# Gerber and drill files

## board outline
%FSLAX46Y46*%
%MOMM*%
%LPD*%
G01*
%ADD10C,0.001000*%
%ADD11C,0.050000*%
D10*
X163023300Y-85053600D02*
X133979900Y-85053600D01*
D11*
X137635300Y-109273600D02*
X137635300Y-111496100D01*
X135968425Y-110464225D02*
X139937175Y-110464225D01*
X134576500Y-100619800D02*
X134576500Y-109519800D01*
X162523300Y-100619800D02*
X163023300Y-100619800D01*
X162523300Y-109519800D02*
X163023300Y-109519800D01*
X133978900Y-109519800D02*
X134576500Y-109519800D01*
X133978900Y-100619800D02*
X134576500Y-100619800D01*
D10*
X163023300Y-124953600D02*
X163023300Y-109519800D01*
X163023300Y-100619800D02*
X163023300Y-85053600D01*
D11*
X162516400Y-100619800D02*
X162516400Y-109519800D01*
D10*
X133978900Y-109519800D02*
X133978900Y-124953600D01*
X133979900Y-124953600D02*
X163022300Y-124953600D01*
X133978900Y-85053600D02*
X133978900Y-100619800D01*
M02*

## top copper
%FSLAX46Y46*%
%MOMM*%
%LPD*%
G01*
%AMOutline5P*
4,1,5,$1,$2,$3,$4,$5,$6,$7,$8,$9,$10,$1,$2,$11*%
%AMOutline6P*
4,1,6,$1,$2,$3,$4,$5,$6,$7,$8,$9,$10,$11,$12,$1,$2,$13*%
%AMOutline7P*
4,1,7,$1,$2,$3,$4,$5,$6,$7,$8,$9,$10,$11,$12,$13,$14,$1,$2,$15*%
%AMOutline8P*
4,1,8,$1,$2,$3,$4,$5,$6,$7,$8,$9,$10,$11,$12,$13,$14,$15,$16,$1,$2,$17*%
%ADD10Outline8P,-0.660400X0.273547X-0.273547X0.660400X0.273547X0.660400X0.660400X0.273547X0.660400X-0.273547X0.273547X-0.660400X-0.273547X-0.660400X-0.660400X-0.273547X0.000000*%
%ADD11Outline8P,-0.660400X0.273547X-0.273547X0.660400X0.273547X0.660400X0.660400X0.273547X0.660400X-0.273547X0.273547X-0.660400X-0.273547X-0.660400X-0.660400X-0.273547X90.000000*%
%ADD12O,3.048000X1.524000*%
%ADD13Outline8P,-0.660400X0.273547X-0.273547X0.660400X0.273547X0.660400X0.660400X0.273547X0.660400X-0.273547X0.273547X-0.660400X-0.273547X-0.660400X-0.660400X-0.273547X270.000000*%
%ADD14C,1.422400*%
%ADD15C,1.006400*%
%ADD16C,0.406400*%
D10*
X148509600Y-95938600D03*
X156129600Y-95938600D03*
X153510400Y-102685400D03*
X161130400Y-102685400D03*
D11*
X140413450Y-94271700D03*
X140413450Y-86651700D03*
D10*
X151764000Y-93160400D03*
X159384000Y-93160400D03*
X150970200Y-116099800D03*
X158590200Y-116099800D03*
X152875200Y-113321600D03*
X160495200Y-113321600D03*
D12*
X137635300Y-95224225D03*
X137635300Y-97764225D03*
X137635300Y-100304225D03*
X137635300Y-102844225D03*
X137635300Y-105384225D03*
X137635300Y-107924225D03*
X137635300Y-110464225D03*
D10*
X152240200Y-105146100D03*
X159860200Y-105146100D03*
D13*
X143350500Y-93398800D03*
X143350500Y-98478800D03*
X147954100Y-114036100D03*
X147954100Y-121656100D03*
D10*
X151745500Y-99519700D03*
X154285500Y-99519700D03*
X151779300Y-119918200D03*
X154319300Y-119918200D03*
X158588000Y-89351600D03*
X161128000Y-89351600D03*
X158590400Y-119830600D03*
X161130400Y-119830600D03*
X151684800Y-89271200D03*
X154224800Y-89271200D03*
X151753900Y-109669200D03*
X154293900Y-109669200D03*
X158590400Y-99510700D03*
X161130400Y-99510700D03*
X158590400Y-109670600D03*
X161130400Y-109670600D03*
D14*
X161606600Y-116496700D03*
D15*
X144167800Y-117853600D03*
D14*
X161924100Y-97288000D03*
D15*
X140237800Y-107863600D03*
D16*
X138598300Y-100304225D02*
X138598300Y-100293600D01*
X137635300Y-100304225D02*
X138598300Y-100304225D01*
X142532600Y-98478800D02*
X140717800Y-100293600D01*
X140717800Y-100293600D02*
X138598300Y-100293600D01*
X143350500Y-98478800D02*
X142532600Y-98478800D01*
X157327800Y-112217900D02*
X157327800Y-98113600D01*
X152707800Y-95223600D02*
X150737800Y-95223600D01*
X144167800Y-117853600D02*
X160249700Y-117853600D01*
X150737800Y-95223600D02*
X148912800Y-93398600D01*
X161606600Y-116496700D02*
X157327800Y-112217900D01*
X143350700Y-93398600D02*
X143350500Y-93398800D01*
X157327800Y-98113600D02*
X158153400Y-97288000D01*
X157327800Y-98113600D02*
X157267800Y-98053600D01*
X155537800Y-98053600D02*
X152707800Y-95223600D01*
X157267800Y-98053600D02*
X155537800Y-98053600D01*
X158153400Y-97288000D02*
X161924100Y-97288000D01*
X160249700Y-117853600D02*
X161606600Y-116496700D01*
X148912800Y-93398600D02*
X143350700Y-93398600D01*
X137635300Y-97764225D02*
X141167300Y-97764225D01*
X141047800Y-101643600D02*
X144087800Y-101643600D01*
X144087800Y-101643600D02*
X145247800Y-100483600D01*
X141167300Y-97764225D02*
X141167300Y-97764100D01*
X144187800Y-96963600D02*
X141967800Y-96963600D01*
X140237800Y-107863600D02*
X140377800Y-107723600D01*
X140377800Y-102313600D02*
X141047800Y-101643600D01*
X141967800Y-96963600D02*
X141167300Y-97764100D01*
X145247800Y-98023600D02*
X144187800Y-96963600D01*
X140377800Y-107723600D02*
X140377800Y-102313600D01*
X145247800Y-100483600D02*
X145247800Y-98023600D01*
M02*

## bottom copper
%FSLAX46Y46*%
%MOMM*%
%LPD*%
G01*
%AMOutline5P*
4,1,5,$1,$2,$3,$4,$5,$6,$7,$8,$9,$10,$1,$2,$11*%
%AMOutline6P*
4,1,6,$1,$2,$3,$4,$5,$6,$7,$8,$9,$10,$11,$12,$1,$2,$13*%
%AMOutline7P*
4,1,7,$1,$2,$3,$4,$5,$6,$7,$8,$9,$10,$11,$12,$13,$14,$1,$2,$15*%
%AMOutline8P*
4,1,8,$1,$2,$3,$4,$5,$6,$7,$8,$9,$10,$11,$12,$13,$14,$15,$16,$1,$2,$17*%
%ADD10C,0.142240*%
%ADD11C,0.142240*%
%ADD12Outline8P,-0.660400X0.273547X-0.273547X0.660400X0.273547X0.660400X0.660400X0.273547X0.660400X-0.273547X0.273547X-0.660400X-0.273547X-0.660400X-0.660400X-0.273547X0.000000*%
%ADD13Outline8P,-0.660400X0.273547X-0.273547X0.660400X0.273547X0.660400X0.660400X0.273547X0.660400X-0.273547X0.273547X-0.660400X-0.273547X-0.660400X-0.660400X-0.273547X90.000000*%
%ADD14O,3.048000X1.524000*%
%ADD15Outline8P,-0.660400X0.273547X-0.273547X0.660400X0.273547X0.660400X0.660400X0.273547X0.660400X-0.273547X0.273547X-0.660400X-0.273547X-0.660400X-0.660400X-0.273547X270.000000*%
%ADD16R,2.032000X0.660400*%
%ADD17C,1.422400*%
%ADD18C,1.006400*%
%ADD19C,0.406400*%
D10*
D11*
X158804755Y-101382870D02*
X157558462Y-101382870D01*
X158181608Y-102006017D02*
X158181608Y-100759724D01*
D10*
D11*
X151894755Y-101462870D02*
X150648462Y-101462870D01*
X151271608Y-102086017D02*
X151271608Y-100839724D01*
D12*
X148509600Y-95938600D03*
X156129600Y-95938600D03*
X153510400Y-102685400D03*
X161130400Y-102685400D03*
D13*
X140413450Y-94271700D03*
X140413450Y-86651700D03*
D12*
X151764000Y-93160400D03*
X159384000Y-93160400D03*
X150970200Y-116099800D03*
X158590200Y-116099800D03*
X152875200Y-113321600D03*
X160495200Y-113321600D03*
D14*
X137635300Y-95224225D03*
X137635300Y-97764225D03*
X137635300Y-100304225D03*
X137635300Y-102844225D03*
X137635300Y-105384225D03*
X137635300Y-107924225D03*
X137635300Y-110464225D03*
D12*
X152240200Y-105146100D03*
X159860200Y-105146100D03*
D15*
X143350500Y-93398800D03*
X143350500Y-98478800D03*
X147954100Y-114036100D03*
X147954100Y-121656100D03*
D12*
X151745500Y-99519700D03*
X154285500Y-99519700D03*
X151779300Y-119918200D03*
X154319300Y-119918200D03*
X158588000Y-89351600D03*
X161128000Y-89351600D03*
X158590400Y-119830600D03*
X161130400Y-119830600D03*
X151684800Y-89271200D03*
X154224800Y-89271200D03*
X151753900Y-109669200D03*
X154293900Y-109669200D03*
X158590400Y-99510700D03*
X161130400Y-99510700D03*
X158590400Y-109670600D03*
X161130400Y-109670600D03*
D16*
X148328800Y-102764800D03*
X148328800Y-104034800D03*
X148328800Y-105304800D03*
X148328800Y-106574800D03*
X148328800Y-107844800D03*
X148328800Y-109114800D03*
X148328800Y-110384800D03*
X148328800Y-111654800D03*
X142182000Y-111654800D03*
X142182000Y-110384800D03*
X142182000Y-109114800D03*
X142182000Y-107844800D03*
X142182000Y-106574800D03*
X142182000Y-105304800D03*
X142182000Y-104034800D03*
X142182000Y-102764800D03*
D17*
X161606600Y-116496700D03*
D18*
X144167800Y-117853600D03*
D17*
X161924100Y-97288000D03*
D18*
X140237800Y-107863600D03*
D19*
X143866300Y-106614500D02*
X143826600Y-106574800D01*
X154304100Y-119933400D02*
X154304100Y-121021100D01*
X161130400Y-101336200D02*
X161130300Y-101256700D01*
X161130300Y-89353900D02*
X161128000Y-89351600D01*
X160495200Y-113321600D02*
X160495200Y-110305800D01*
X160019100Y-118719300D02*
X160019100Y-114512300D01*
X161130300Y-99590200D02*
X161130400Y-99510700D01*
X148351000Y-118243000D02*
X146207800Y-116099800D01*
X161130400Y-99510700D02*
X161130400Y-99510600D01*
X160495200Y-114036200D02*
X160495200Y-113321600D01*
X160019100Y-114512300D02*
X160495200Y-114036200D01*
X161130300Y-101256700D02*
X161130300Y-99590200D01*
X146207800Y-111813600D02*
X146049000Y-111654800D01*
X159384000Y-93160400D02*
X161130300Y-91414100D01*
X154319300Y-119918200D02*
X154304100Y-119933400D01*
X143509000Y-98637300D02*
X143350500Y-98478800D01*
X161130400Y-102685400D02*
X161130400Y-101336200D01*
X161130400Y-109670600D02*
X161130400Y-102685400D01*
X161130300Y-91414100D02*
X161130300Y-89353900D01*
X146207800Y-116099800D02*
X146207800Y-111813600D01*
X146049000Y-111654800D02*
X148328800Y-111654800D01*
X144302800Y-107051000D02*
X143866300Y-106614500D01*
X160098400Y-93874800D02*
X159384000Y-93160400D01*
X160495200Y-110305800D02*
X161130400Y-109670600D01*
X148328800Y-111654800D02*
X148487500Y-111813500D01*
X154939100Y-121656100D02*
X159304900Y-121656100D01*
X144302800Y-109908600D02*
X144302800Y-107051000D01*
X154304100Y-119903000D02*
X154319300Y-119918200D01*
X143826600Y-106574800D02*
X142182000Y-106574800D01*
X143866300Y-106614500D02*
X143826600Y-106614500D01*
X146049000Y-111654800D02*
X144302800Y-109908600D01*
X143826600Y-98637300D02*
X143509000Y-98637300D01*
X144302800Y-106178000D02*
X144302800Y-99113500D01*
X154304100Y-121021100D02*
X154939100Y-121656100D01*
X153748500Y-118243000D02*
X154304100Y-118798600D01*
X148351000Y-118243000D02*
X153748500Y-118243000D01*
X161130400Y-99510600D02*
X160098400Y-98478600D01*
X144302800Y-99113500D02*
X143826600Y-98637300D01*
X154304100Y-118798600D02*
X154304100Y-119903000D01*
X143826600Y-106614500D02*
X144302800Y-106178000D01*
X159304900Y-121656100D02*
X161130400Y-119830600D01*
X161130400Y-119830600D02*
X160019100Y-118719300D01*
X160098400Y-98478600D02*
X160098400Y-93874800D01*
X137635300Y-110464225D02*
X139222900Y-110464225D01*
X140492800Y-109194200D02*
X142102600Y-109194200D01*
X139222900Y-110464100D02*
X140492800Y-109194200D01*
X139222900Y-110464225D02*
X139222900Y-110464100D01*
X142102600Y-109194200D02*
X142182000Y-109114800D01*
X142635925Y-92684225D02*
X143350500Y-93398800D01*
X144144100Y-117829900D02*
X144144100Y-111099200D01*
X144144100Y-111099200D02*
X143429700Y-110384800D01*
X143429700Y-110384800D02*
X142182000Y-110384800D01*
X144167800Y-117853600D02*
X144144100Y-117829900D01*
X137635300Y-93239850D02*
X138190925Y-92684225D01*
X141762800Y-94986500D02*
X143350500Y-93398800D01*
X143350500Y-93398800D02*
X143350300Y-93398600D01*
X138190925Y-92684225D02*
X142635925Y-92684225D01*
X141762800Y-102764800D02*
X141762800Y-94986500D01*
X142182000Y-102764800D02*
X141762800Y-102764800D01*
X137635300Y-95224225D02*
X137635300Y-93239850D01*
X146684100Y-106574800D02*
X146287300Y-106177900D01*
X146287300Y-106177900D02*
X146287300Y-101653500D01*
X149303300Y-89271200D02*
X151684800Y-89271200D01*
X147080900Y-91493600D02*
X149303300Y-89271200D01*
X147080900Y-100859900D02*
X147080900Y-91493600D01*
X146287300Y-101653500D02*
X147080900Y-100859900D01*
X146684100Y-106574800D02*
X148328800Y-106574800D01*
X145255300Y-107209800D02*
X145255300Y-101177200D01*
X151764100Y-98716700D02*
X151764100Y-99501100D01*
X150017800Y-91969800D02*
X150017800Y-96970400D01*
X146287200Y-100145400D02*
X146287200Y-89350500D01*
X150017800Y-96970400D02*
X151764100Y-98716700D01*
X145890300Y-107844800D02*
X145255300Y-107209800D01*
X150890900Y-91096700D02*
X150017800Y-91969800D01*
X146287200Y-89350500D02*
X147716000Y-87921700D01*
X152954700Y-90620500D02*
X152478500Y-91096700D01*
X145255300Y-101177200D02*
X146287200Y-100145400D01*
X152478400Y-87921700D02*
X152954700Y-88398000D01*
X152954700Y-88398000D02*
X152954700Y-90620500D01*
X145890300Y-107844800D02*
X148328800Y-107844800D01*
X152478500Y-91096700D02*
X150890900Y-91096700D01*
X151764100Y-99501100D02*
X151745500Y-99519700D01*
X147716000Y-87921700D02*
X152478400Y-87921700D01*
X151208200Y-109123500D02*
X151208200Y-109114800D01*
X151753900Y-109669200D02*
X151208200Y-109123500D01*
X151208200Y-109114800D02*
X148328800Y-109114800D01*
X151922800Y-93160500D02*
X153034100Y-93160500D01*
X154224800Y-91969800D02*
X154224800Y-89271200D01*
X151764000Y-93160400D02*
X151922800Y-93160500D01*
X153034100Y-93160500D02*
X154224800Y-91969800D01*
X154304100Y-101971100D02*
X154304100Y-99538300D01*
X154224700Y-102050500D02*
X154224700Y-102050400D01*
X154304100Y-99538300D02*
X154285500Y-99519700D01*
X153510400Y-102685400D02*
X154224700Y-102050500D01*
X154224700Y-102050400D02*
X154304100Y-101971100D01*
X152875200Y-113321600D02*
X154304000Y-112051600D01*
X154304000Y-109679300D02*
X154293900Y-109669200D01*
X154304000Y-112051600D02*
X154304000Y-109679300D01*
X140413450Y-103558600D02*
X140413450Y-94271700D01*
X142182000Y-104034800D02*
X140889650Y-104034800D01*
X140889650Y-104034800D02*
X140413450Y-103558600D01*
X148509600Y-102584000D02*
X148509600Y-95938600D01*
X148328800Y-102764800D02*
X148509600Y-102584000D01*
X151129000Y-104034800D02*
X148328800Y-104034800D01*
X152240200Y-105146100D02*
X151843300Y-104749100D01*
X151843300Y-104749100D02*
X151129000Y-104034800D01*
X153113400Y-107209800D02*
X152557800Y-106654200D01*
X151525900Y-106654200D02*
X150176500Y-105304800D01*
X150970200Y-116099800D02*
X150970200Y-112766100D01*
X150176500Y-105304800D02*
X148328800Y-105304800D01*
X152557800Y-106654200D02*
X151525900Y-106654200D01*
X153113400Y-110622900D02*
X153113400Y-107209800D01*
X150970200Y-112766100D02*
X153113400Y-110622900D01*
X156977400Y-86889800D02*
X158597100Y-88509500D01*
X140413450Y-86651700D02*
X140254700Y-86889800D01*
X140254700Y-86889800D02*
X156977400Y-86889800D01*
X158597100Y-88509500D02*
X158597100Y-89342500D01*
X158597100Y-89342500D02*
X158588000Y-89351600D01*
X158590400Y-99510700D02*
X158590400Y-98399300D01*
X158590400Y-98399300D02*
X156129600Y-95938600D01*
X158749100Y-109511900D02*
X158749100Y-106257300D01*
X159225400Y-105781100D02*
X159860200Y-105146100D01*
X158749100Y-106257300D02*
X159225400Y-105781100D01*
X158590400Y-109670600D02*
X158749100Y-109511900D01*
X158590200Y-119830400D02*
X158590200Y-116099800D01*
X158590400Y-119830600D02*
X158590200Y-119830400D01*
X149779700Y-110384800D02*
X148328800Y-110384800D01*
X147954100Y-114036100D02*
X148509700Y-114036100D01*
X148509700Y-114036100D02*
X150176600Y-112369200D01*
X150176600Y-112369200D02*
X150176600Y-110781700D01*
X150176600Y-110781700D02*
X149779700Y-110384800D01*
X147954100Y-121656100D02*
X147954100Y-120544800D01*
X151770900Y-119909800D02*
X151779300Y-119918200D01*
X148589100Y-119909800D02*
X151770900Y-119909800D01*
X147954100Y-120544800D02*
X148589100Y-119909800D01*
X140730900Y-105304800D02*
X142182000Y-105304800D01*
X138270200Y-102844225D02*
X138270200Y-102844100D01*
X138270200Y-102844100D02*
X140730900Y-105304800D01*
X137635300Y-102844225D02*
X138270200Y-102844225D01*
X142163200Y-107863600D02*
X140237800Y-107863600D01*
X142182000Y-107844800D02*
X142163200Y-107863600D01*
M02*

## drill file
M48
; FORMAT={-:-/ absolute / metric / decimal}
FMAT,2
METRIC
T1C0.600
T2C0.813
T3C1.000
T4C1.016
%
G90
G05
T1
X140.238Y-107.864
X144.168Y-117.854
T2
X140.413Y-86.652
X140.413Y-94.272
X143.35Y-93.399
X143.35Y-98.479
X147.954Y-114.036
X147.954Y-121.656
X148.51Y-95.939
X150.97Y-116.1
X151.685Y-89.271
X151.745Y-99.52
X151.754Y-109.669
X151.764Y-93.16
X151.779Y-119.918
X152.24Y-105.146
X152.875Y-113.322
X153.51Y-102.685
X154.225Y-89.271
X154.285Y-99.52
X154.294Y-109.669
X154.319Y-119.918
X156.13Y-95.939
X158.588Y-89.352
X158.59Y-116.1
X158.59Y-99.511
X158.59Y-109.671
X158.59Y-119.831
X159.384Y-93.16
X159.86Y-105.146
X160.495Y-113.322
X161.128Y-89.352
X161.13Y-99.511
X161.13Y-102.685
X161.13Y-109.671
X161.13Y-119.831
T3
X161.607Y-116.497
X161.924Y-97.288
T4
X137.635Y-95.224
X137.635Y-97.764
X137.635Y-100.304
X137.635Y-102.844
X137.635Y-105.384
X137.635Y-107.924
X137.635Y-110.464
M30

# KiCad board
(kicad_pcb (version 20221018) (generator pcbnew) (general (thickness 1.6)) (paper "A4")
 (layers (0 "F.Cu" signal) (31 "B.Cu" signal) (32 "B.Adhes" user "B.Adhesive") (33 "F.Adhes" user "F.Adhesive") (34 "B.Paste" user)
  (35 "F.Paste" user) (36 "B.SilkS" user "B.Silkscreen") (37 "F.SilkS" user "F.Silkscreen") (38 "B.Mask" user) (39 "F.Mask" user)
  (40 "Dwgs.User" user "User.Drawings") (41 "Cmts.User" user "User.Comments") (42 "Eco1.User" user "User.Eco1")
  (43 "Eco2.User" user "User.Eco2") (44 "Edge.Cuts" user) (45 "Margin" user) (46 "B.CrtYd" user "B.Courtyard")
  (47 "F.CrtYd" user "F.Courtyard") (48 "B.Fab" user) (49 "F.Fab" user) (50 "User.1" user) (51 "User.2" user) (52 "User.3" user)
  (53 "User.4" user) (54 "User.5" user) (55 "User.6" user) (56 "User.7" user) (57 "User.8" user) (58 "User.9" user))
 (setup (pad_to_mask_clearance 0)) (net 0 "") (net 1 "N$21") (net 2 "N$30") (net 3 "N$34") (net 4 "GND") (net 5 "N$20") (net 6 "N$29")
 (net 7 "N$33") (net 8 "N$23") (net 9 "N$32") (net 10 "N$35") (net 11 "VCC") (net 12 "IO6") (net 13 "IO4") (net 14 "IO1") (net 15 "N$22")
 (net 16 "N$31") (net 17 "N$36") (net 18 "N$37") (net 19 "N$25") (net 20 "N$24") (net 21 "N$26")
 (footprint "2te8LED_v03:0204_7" (layer "F.Cu") (at 152.3196 95.9386)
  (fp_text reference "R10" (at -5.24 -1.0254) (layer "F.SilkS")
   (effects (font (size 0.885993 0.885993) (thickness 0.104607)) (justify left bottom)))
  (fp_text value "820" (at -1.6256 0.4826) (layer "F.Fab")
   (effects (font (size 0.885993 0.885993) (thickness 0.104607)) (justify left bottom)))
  (pad "1" thru_hole roundrect (at -3.81 0) (size 1.3208 1.3208) (drill 0.8128) (layers "*.Cu" "*.Mask") (roundrect_rratio 0.25)
   (chamfer_ratio 0.2928932188) (chamfer top_left top_right bottom_left bottom_right) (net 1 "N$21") (solder_mask_margin 0.1016)
   (thermal_bridge_angle 0))
  (pad "2" thru_hole roundrect (at 3.81 0) (size 1.3208 1.3208) (drill 0.8128) (layers "*.Cu" "*.Mask") (roundrect_rratio 0.25)
   (chamfer_ratio 0.2928932188) (chamfer top_left top_right bottom_left bottom_right) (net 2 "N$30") (solder_mask_margin 0.1016)
   (thermal_bridge_angle 0)))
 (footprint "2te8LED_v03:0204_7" (layer "F.Cu") (at 157.3204 102.6854)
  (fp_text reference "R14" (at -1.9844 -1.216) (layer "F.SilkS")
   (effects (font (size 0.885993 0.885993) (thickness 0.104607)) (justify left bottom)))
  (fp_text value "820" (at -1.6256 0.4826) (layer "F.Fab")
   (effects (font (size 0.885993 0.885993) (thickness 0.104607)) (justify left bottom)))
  (pad "1" thru_hole roundrect (at -3.81 0) (size 1.3208 1.3208) (drill 0.8128) (layers "*.Cu" "*.Mask") (roundrect_rratio 0.25)
   (chamfer_ratio 0.2928932188) (chamfer top_left top_right bottom_left bottom_right) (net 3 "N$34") (solder_mask_margin 0.1016)
   (thermal_bridge_angle 0))
  (pad "2" thru_hole roundrect (at 3.81 0) (size 1.3208 1.3208) (drill 0.8128) (layers "*.Cu" "*.Mask") (roundrect_rratio 0.25)
   (chamfer_ratio 0.2928932188) (chamfer top_left top_right bottom_left bottom_right) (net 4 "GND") (solder_mask_margin 0.1016)
   (thermal_bridge_angle 0)))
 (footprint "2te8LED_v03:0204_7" (layer "F.Cu") (at 140.41345 90.4617 90)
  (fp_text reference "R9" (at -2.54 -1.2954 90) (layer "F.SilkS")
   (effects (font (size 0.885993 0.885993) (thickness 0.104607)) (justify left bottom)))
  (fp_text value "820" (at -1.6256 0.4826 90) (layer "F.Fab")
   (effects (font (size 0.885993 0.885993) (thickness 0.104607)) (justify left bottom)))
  (pad "1" thru_hole roundrect (at -3.81 0 90) (size 1.3208 1.3208) (drill 0.8128) (layers "*.Cu" "*.Mask") (roundrect_rratio 0.25)
   (chamfer_ratio 0.2928932188) (chamfer top_left top_right bottom_left bottom_right) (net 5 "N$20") (solder_mask_margin 0.1016)
   (thermal_bridge_angle 0))
  (pad "2" thru_hole roundrect (at 3.81 0 90) (size 1.3208 1.3208) (drill 0.8128) (layers "*.Cu" "*.Mask") (roundrect_rratio 0.25)
   (chamfer_ratio 0.2928932188) (chamfer top_left top_right bottom_left bottom_right) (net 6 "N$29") (solder_mask_margin 0.1016)
   (thermal_bridge_angle 0)))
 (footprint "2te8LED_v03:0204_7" (layer "F.Cu") (at 155.574 93.1604)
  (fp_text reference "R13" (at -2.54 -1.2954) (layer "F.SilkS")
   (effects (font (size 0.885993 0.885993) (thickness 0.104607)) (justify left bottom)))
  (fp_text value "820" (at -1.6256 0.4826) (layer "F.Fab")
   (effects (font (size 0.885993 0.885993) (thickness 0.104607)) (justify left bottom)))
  (pad "1" thru_hole roundrect (at -3.81 0) (size 1.3208 1.3208) (drill 0.8128) (layers "*.Cu" "*.Mask") (roundrect_rratio 0.25)
   (chamfer_ratio 0.2928932188) (chamfer top_left top_right bottom_left bottom_right) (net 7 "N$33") (solder_mask_margin 0.1016)
   (thermal_bridge_angle 0))
  (pad "2" thru_hole roundrect (at 3.81 0) (size 1.3208 1.3208) (drill 0.8128) (layers "*.Cu" "*.Mask") (roundrect_rratio 0.25)
   (chamfer_ratio 0.2928932188) (chamfer top_left top_right bottom_left bottom_right) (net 4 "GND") (solder_mask_margin 0.1016)
   (thermal_bridge_angle 0)))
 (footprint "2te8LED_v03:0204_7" (layer "F.Cu") (at 154.7802 116.0998)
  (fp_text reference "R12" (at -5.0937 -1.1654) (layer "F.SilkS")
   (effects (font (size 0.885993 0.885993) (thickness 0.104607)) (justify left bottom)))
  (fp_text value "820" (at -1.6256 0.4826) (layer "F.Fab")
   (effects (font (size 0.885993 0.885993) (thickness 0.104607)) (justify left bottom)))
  (pad "1" thru_hole roundrect (at -3.81 0) (size 1.3208 1.3208) (drill 0.8128) (layers "*.Cu" "*.Mask") (roundrect_rratio 0.25)
   (chamfer_ratio 0.2928932188) (chamfer top_left top_right bottom_left bottom_right) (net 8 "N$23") (solder_mask_margin 0.1016)
   (thermal_bridge_angle 0))
  (pad "2" thru_hole roundrect (at 3.81 0) (size 1.3208 1.3208) (drill 0.8128) (layers "*.Cu" "*.Mask") (roundrect_rratio 0.25)
   (chamfer_ratio 0.2928932188) (chamfer top_left top_right bottom_left bottom_right) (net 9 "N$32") (solder_mask_margin 0.1016)
   (thermal_bridge_angle 0)))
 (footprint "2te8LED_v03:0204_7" (layer "F.Cu") (at 156.6852 113.3216)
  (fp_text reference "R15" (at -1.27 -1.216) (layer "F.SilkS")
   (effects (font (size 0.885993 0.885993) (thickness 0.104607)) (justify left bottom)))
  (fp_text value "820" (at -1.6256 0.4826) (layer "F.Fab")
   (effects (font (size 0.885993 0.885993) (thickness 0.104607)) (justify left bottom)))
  (pad "1" thru_hole roundrect (at -3.81 0) (size 1.3208 1.3208) (drill 0.8128) (layers "*.Cu" "*.Mask") (roundrect_rratio 0.25)
   (chamfer_ratio 0.2928932188) (chamfer top_left top_right bottom_left bottom_right) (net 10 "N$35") (solder_mask_margin 0.1016)
   (thermal_bridge_angle 0))
  (pad "2" thru_hole roundrect (at 3.81 0) (size 1.3208 1.3208) (drill 0.8128) (layers "*.Cu" "*.Mask") (roundrect_rratio 0.25)
   (chamfer_ratio 0.2928932188) (chamfer top_left top_right bottom_left bottom_right) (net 4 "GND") (solder_mask_margin 0.1016)
   (thermal_bridge_angle 0)))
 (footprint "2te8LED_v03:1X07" (layer "F.Cu") (at 137.6353 102.844225 -90)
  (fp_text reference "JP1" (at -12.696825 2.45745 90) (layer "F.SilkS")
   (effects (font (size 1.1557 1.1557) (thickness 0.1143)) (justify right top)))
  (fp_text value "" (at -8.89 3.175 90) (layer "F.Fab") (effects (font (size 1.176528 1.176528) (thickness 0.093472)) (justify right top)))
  (pad "1" thru_hole oval (at -7.62 0) (size 3.048 1.524) (drill 1.016) (layers "*.Cu" "*.Mask") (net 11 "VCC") (solder_mask_margin 0.1016)
   (thermal_bridge_angle 0))
  (pad "2" thru_hole oval (at -5.08 0) (size 3.048 1.524) (drill 1.016) (layers "*.Cu" "*.Mask") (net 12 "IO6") (solder_mask_margin 0.1016)
   (thermal_bridge_angle 0))
  (pad "3" thru_hole oval (at -2.54 0) (size 3.048 1.524) (drill 1.016) (layers "*.Cu" "*.Mask") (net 4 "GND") (solder_mask_margin 0.1016)
   (thermal_bridge_angle 0))
  (pad "4" thru_hole oval (at 0 0) (size 3.048 1.524) (drill 1.016) (layers "*.Cu" "*.Mask") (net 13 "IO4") (solder_mask_margin 0.1016)
   (thermal_bridge_angle 0))
  (pad "5" thru_hole oval (at 2.54 0) (size 3.048 1.524) (drill 1.016) (layers "*.Cu" "*.Mask") (solder_mask_margin 0.1016)
   (thermal_bridge_angle 0))
  (pad "6" thru_hole oval (at 5.08 0) (size 3.048 1.524) (drill 1.016) (layers "*.Cu" "*.Mask") (solder_mask_margin 0.1016)
   (thermal_bridge_angle 0))
  (pad "7" thru_hole oval (at 7.62 0) (size 3.048 1.524) (drill 1.016) (layers "*.Cu" "*.Mask") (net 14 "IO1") (solder_mask_margin 0.1016)
   (thermal_bridge_angle 0)))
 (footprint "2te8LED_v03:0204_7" (layer "F.Cu") (at 156.0502 105.1461)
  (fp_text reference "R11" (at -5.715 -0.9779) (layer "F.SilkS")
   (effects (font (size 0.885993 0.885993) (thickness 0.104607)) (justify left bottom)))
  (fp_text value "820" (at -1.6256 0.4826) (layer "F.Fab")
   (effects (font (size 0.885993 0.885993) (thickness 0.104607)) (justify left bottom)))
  (pad "1" thru_hole roundrect (at -3.81 0) (size 1.3208 1.3208) (drill 0.8128) (layers "*.Cu" "*.Mask") (roundrect_rratio 0.25)
   (chamfer_ratio 0.2928932188) (chamfer top_left top_right bottom_left bottom_right) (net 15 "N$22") (solder_mask_margin 0.1016)
   (thermal_bridge_angle 0))
  (pad "2" thru_hole roundrect (at 3.81 0) (size 1.3208 1.3208) (drill 0.8128) (layers "*.Cu" "*.Mask") (roundrect_rratio 0.25)
   (chamfer_ratio 0.2928932188) (chamfer top_left top_right bottom_left bottom_right) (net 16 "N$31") (solder_mask_margin 0.1016)
   (thermal_bridge_angle 0)))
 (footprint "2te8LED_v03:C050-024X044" (layer "F.Cu") (at 143.3505 95.9388 -90)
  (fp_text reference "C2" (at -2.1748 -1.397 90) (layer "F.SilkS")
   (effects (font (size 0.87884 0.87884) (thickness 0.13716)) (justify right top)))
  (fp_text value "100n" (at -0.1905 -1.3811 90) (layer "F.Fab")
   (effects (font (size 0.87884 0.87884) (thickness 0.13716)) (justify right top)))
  (pad "1" thru_hole roundrect (at -2.54 0 270) (size 1.3208 1.3208) (drill 0.8128) (layers "*.Cu" "*.Mask") (roundrect_rratio 0.25)
   (chamfer_ratio 0.2928932188) (chamfer top_left top_right bottom_left bottom_right) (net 11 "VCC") (solder_mask_margin 0.1016)
   (thermal_bridge_angle 0))
  (pad "2" thru_hole roundrect (at 2.54 0 270) (size 1.3208 1.3208) (drill 0.8128) (layers "*.Cu" "*.Mask") (roundrect_rratio 0.25)
   (chamfer_ratio 0.2928932188) (chamfer top_left top_right bottom_left bottom_right) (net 4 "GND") (solder_mask_margin 0.1016)
   (thermal_bridge_angle 0)))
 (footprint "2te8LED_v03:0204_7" (layer "F.Cu") (at 147.9541 117.8461 -90)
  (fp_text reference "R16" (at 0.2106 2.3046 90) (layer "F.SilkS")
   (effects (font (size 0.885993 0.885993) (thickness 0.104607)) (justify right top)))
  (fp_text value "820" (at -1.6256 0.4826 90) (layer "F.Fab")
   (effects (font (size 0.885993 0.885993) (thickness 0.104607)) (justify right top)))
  (pad "1" thru_hole roundrect (at -3.81 0 270) (size 1.3208 1.3208) (drill 0.8128) (layers "*.Cu" "*.Mask") (roundrect_rratio 0.25)
   (chamfer_ratio 0.2928932188) (chamfer top_left top_right bottom_left bottom_right) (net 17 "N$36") (solder_mask_margin 0.1016)
   (thermal_bridge_angle 0))
  (pad "2" thru_hole roundrect (at 3.81 0 270) (size 1.3208 1.3208) (drill 0.8128) (layers "*.Cu" "*.Mask") (roundrect_rratio 0.25)
   (chamfer_ratio 0.2928932188) (chamfer top_left top_right bottom_left bottom_right) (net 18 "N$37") (solder_mask_margin 0.1016)
   (thermal_bridge_angle 0)))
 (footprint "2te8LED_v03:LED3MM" (layer "B.Cu") (at 153.0155 99.5197)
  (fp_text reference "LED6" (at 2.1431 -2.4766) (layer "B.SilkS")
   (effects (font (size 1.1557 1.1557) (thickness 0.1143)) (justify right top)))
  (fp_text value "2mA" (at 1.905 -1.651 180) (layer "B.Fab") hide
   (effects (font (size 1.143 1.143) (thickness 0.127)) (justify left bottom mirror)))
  (pad "A" thru_hole roundrect (at -1.27 0) (size 1.3208 1.3208) (drill 0.8128) (layers "*.Cu" "*.Mask") (roundrect_rratio 0.25)
   (chamfer_ratio 0.2928932188) (chamfer top_left top_right bottom_left bottom_right) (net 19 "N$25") (solder_mask_margin 0.1016)
   (thermal_bridge_angle 0))
  (pad "K" thru_hole roundrect (at 1.27 0) (size 1.3208 1.3208) (drill 0.8128) (layers "*.Cu" "*.Mask") (roundrect_rratio 0.25)
   (chamfer_ratio 0.2928932188) (chamfer top_left top_right bottom_left bottom_right) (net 3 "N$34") (solder_mask_margin 0.1016)
   (thermal_bridge_angle 0)))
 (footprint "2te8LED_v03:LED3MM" (layer "B.Cu") (at 153.0493 119.9182)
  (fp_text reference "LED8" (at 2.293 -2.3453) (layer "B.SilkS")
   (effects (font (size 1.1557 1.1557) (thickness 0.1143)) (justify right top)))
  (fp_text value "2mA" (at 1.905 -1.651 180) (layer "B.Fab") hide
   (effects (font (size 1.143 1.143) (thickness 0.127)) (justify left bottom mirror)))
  (pad "A" thru_hole roundrect (at -1.27 0) (size 1.3208 1.3208) (drill 0.8128) (layers "*.Cu" "*.Mask") (roundrect_rratio 0.25)
   (chamfer_ratio 0.2928932188) (chamfer top_left top_right bottom_left bottom_right) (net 18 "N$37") (solder_mask_margin 0.1016)
   (thermal_bridge_angle 0))
  (pad "K" thru_hole roundrect (at 1.27 0) (size 1.3208 1.3208) (drill 0.8128) (layers "*.Cu" "*.Mask") (roundrect_rratio 0.25)
   (chamfer_ratio 0.2928932188) (chamfer top_left top_right bottom_left bottom_right) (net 4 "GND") (solder_mask_margin 0.1016)
   (thermal_bridge_angle 0)))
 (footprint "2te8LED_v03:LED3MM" (layer "B.Cu") (at 159.858 89.3516)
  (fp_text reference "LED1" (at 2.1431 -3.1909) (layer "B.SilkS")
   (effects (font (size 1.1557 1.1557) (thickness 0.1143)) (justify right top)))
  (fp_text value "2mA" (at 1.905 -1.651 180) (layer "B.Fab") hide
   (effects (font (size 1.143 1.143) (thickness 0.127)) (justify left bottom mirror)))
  (pad "A" thru_hole roundrect (at -1.27 0) (size 1.3208 1.3208) (drill 0.8128) (layers "*.Cu" "*.Mask") (roundrect_rratio 0.25)
   (chamfer_ratio 0.2928932188) (chamfer top_left top_right bottom_left bottom_right) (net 6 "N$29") (solder_mask_margin 0.1016)
   (thermal_bridge_angle 0))
  (pad "K" thru_hole roundrect (at 1.27 0) (size 1.3208 1.3208) (drill 0.8128) (layers "*.Cu" "*.Mask") (roundrect_rratio 0.25)
   (chamfer_ratio 0.2928932188) (chamfer top_left top_right bottom_left bottom_right) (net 4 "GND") (solder_mask_margin 0.1016)
   (thermal_bridge_angle 0)))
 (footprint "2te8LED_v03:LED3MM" (layer "B.Cu") (at 159.8604 119.8306)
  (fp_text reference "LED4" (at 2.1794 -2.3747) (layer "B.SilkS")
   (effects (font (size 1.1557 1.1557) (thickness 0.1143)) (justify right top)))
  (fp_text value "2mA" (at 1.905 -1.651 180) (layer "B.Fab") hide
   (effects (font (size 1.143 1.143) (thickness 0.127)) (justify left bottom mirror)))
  (pad "A" thru_hole roundrect (at -1.27 0) (size 1.3208 1.3208) (drill 0.8128) (layers "*.Cu" "*.Mask") (roundrect_rratio 0.25)
   (chamfer_ratio 0.2928932188) (chamfer top_left top_right bottom_left bottom_right) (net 9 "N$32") (solder_mask_margin 0.1016)
   (thermal_bridge_angle 0))
  (pad "K" thru_hole roundrect (at 1.27 0) (size 1.3208 1.3208) (drill 0.8128) (layers "*.Cu" "*.Mask") (roundrect_rratio 0.25)
   (chamfer_ratio 0.2928932188) (chamfer top_left top_right bottom_left bottom_right) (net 4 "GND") (solder_mask_margin 0.1016)
   (thermal_bridge_angle 0)))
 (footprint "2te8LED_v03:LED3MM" (layer "B.Cu") (at 152.9548 89.2712)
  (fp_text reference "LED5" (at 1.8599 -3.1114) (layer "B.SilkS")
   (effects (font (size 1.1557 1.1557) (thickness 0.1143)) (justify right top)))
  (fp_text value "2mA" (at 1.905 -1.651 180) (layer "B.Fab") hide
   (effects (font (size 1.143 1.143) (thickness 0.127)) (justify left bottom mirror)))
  (pad "A" thru_hole roundrect (at -1.27 0) (size 1.3208 1.3208) (drill 0.8128) (layers "*.Cu" "*.Mask") (roundrect_rratio 0.25)
   (chamfer_ratio 0.2928932188) (chamfer top_left top_right bottom_left bottom_right) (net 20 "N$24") (solder_mask_margin 0.1016)
   (thermal_bridge_angle 0))
  (pad "K" thru_hole roundrect (at 1.27 0) (size 1.3208 1.3208) (drill 0.8128) (layers "*.Cu" "*.Mask") (roundrect_rratio 0.25)
   (chamfer_ratio 0.2928932188) (chamfer top_left top_right bottom_left bottom_right) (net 7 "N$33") (solder_mask_margin 0.1016)
   (thermal_bridge_angle 0)))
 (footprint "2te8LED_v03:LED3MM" (layer "B.Cu") (at 153.0239 109.6692)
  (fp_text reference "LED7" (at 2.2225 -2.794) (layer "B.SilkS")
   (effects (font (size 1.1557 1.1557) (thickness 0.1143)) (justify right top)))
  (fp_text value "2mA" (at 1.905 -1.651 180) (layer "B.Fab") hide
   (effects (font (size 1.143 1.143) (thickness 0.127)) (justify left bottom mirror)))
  (pad "A" thru_hole roundrect (at -1.27 0) (size 1.3208 1.3208) (drill 0.8128) (layers "*.Cu" "*.Mask") (roundrect_rratio 0.25)
   (chamfer_ratio 0.2928932188) (chamfer top_left top_right bottom_left bottom_right) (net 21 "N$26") (solder_mask_margin 0.1016)
   (thermal_bridge_angle 0))
  (pad "K" thru_hole roundrect (at 1.27 0) (size 1.3208 1.3208) (drill 0.8128) (layers "*.Cu" "*.Mask") (roundrect_rratio 0.25)
   (chamfer_ratio 0.2928932188) (chamfer top_left top_right bottom_left bottom_right) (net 10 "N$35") (solder_mask_margin 0.1016)
   (thermal_bridge_angle 0)))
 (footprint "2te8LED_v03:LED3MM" (layer "B.Cu") (at 159.8604 99.5107)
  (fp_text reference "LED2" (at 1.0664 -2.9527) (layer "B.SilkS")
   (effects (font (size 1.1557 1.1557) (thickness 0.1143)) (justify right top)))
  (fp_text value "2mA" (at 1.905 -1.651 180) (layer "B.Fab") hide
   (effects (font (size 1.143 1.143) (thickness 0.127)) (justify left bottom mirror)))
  (pad "A" thru_hole roundrect (at -1.27 0) (size 1.3208 1.3208) (drill 0.8128) (layers "*.Cu" "*.Mask") (roundrect_rratio 0.25)
   (chamfer_ratio 0.2928932188) (chamfer top_left top_right bottom_left bottom_right) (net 2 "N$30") (solder_mask_margin 0.1016)
   (thermal_bridge_angle 0))
  (pad "K" thru_hole roundrect (at 1.27 0) (size 1.3208 1.3208) (drill 0.8128) (layers "*.Cu" "*.Mask") (roundrect_rratio 0.25)
   (chamfer_ratio 0.2928932188) (chamfer top_left top_right bottom_left bottom_right) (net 4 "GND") (solder_mask_margin 0.1016)
   (thermal_bridge_angle 0)))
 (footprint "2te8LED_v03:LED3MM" (layer "B.Cu") (at 159.8604 109.6706)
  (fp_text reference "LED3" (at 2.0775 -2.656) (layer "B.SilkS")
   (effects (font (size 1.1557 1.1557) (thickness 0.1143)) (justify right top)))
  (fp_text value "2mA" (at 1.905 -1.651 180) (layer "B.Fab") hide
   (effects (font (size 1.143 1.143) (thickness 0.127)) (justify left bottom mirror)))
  (pad "A" thru_hole roundrect (at -1.27 0) (size 1.3208 1.3208) (drill 0.8128) (layers "*.Cu" "*.Mask") (roundrect_rratio 0.25)
   (chamfer_ratio 0.2928932188) (chamfer top_left top_right bottom_left bottom_right) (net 16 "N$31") (solder_mask_margin 0.1016)
   (thermal_bridge_angle 0))
  (pad "K" thru_hole roundrect (at 1.27 0) (size 1.3208 1.3208) (drill 0.8128) (layers "*.Cu" "*.Mask") (roundrect_rratio 0.25)
   (chamfer_ratio 0.2928932188) (chamfer top_left top_right bottom_left bottom_right) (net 4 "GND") (solder_mask_margin 0.1016)
   (thermal_bridge_angle 0)))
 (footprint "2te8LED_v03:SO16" (layer "B.Cu") (at 145.2554 107.2098 -90)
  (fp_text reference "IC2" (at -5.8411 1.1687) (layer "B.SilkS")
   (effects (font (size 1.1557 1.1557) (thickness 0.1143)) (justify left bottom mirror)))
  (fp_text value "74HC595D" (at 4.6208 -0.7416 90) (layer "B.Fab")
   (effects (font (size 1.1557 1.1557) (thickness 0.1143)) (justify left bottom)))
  (pad "1" smd rect (at -4.445 -3.0734 270) (size 0.6604 2.032) (layers "B.Cu" "B.Paste" "B.Mask") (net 1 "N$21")
   (solder_mask_margin 0.1016) (thermal_bridge_angle 0))
  (pad "2" smd rect (at -3.175 -3.0734 270) (size 0.6604 2.032) (layers "B.Cu" "B.Paste" "B.Mask") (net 15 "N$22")
   (solder_mask_margin 0.1016) (thermal_bridge_angle 0))
  (pad "3" smd rect (at -1.905 -3.0734 270) (size 0.6604 2.032) (layers "B.Cu" "B.Paste" "B.Mask") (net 8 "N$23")
   (solder_mask_margin 0.1016) (thermal_bridge_angle 0))
  (pad "4" smd rect (at -0.635 -3.0734 270) (size 0.6604 2.032) (layers "B.Cu" "B.Paste" "B.Mask") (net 20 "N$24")
   (solder_mask_margin 0.1016) (thermal_bridge_angle 0))
  (pad "5" smd rect (at 0.635 -3.0734 270) (size 0.6604 2.032) (layers "B.Cu" "B.Paste" "B.Mask") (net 19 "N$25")
   (solder_mask_margin 0.1016) (thermal_bridge_angle 0))
  (pad "6" smd rect (at 1.905 -3.0734 270) (size 0.6604 2.032) (layers "B.Cu" "B.Paste" "B.Mask") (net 21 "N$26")
   (solder_mask_margin 0.1016) (thermal_bridge_angle 0))
  (pad "7" smd rect (at 3.175 -3.0734 270) (size 0.6604 2.032) (layers "B.Cu" "B.Paste" "B.Mask") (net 17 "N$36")
   (solder_mask_margin 0.1016) (thermal_bridge_angle 0))
  (pad "8" smd rect (at 4.445 -3.0734 270) (size 0.6604 2.032) (layers "B.Cu" "B.Paste" "B.Mask") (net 4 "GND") (solder_mask_margin 0.1016)
   (thermal_bridge_angle 0))
  (pad "9" smd rect (at 4.445 3.0734 270) (size 0.6604 2.032) (layers "B.Cu" "B.Paste" "B.Mask") (solder_mask_margin 0.1016)
   (thermal_bridge_angle 0))
  (pad "10" smd rect (at 3.175 3.0734 270) (size 0.6604 2.032) (layers "B.Cu" "B.Paste" "B.Mask") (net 11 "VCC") (solder_mask_margin 0.1016)
   (thermal_bridge_angle 0))
  (pad "11" smd rect (at 1.905 3.0734 270) (size 0.6604 2.032) (layers "B.Cu" "B.Paste" "B.Mask") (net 14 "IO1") (solder_mask_margin 0.1016)
   (thermal_bridge_angle 0))
  (pad "12" smd rect (at 0.635 3.0734 270) (size 0.6604 2.032) (layers "B.Cu" "B.Paste" "B.Mask") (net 12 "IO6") (solder_mask_margin 0.1016)
   (thermal_bridge_angle 0))
  (pad "13" smd rect (at -0.635 3.0734 270) (size 0.6604 2.032) (layers "B.Cu" "B.Paste" "B.Mask") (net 4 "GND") (solder_mask_margin 0.1016)
   (thermal_bridge_angle 0))
  (pad "14" smd rect (at -1.905 3.0734 270) (size 0.6604 2.032) (layers "B.Cu" "B.Paste" "B.Mask") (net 13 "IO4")
   (solder_mask_margin 0.1016) (thermal_bridge_angle 0))
  (pad "15" smd rect (at -3.175 3.0734 270) (size 0.6604 2.032) (layers "B.Cu" "B.Paste" "B.Mask") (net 5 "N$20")
   (solder_mask_margin 0.1016) (thermal_bridge_angle 0))
  (pad "16" smd rect (at -4.445 3.0734 270) (size 0.6604 2.032) (layers "B.Cu" "B.Paste" "B.Mask") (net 11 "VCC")
   (solder_mask_margin 0.1016) (thermal_bridge_angle 0)))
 (gr_line (start 163.0233 85.0536) (end 133.9799 85.0536) (stroke (width 0.001) (type solid)) (layer "Edge.Cuts"))
 (gr_line (start 137.6353 109.2736) (end 137.6353 111.4961) (stroke (width 0.05) (type solid)) (layer "Edge.Cuts"))
 (gr_line (start 135.968425 110.464225) (end 139.937175 110.464225) (stroke (width 0.05) (type solid)) (layer "Edge.Cuts"))
 (gr_line (start 134.5765 100.6198) (end 134.5765 109.5198) (stroke (width 0.05) (type solid)) (layer "Edge.Cuts"))
 (gr_line (start 162.5233 100.6198) (end 163.0233 100.6198) (stroke (width 0.05) (type solid)) (layer "Edge.Cuts"))
 (gr_line (start 162.5233 109.5198) (end 163.0233 109.5198) (stroke (width 0.05) (type solid)) (layer "Edge.Cuts"))
 (gr_line (start 133.9789 109.5198) (end 134.5765 109.5198) (stroke (width 0.05) (type solid)) (layer "Edge.Cuts"))
 (gr_line (start 133.9789 100.6198) (end 134.5765 100.6198) (stroke (width 0.05) (type solid)) (layer "Edge.Cuts"))
 (gr_line (start 163.0233 124.9536) (end 163.0233 109.5198) (stroke (width 0.001) (type solid)) (layer "Edge.Cuts"))
 (gr_line (start 163.0233 100.6198) (end 163.0233 85.0536) (stroke (width 0.001) (type solid)) (layer "Edge.Cuts"))
 (gr_line (start 162.5164 100.6198) (end 162.5164 109.5198) (stroke (width 0.05) (type solid)) (layer "Edge.Cuts"))
 (gr_line (start 133.9789 109.5198) (end 133.9789 124.9536) (stroke (width 0.001) (type solid)) (layer "Edge.Cuts"))
 (gr_line (start 133.9799 124.9536) (end 163.0223 124.9536) (stroke (width 0.001) (type solid)) (layer "Edge.Cuts"))
 (gr_line (start 133.9789 85.0536) (end 133.9789 100.6198) (stroke (width 0.001) (type solid)) (layer "Edge.Cuts"))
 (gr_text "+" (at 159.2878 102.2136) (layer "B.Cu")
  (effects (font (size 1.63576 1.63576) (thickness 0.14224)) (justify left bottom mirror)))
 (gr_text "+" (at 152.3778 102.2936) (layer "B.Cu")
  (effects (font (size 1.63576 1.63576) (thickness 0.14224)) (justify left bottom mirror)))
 (segment (start 138.5983 100.304225) (end 138.5983 100.2936) (width 0.4064) (layer "F.Cu") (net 4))
 (segment (start 137.6353 100.304225) (end 138.5983 100.304225) (width 0.4064) (layer "F.Cu") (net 4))
 (segment (start 142.5326 98.4788) (end 140.7178 100.2936) (width 0.4064) (layer "F.Cu") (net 4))
 (segment (start 140.7178 100.2936) (end 138.5983 100.2936) (width 0.4064) (layer "F.Cu") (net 4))
 (segment (start 143.3505 98.4788) (end 142.5326 98.4788) (width 0.4064) (layer "F.Cu") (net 4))
 (segment (start 143.8663 106.6145) (end 143.8266 106.5748) (width 0.4064) (layer "B.Cu") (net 4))
 (segment (start 154.3041 119.9334) (end 154.3041 121.0211) (width 0.4064) (layer "B.Cu") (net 4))
 (segment (start 161.1304 101.3362) (end 161.1303 101.2567) (width 0.4064) (layer "B.Cu") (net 4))
 (segment (start 161.1303 89.3539) (end 161.128 89.3516) (width 0.4064) (layer "B.Cu") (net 4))
 (segment (start 160.4952 113.3216) (end 160.4952 110.3058) (width 0.4064) (layer "B.Cu") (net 4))
 (segment (start 160.0191 118.7193) (end 160.0191 114.5123) (width 0.4064) (layer "B.Cu") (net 4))
 (segment (start 161.1303 99.5902) (end 161.1304 99.5107) (width 0.4064) (layer "B.Cu") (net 4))
 (segment (start 148.351 118.243) (end 146.2078 116.0998) (width 0.4064) (layer "B.Cu") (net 4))
 (segment (start 161.1304 99.5107) (end 161.1304 99.5106) (width 0.4064) (layer "B.Cu") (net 4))
 (segment (start 160.4952 114.0362) (end 160.4952 113.3216) (width 0.4064) (layer "B.Cu") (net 4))
 (segment (start 160.0191 114.5123) (end 160.4952 114.0362) (width 0.4064) (layer "B.Cu") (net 4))
 (segment (start 161.1303 101.2567) (end 161.1303 99.5902) (width 0.4064) (layer "B.Cu") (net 4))
 (segment (start 146.2078 111.8136) (end 146.049 111.6548) (width 0.4064) (layer "B.Cu") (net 4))
 (segment (start 159.384 93.1604) (end 161.1303 91.4141) (width 0.4064) (layer "B.Cu") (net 4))
 (segment (start 154.3193 119.9182) (end 154.3041 119.9334) (width 0.4064) (layer "B.Cu") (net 4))
 (segment (start 143.509 98.6373) (end 143.3505 98.4788) (width 0.4064) (layer "B.Cu") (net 4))
 (segment (start 161.1304 102.6854) (end 161.1304 101.3362) (width 0.4064) (layer "B.Cu") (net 4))
 (segment (start 161.1304 109.6706) (end 161.1304 102.6854) (width 0.4064) (layer "B.Cu") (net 4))
 (segment (start 161.1303 91.4141) (end 161.1303 89.3539) (width 0.4064) (layer "B.Cu") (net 4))
 (segment (start 146.2078 116.0998) (end 146.2078 111.8136) (width 0.4064) (layer "B.Cu") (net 4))
 (segment (start 146.049 111.6548) (end 148.3288 111.6548) (width 0.4064) (layer "B.Cu") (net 4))
 (segment (start 144.3028 107.051) (end 143.8663 106.6145) (width 0.4064) (layer "B.Cu") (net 4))
 (segment (start 160.0984 93.8748) (end 159.384 93.1604) (width 0.4064) (layer "B.Cu") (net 4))
 (segment (start 160.4952 110.3058) (end 161.1304 109.6706) (width 0.4064) (layer "B.Cu") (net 4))
 (segment (start 148.3288 111.6548) (end 148.4875 111.8135) (width 0.4064) (layer "B.Cu") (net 4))
 (segment (start 154.9391 121.6561) (end 159.3049 121.6561) (width 0.4064) (layer "B.Cu") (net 4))
 (segment (start 144.3028 109.9086) (end 144.3028 107.051) (width 0.4064) (layer "B.Cu") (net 4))
 (segment (start 154.3041 119.903) (end 154.3193 119.9182) (width 0.4064) (layer "B.Cu") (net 4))
 (segment (start 143.8266 106.5748) (end 142.182 106.5748) (width 0.4064) (layer "B.Cu") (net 4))
 (segment (start 143.8663 106.6145) (end 143.8266 106.6145) (width 0.4064) (layer "B.Cu") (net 4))
 (segment (start 146.049 111.6548) (end 144.3028 109.9086) (width 0.4064) (layer "B.Cu") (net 4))
 (segment (start 143.8266 98.6373) (end 143.509 98.6373) (width 0.4064) (layer "B.Cu") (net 4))
 (segment (start 144.3028 106.178) (end 144.3028 99.1135) (width 0.4064) (layer "B.Cu") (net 4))
 (segment (start 154.3041 121.0211) (end 154.9391 121.6561) (width 0.4064) (layer "B.Cu") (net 4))
 (segment (start 153.7485 118.243) (end 154.3041 118.7986) (width 0.4064) (layer "B.Cu") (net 4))
 (segment (start 148.351 118.243) (end 153.7485 118.243) (width 0.4064) (layer "B.Cu") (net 4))
 (segment (start 161.1304 99.5106) (end 160.0984 98.4786) (width 0.4064) (layer "B.Cu") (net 4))
 (segment (start 144.3028 99.1135) (end 143.8266 98.6373) (width 0.4064) (layer "B.Cu") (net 4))
 (segment (start 154.3041 118.7986) (end 154.3041 119.903) (width 0.4064) (layer "B.Cu") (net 4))
 (segment (start 143.8266 106.6145) (end 144.3028 106.178) (width 0.4064) (layer "B.Cu") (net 4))
 (segment (start 159.3049 121.6561) (end 161.1304 119.8306) (width 0.4064) (layer "B.Cu") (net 4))
 (segment (start 161.1304 119.8306) (end 160.0191 118.7193) (width 0.4064) (layer "B.Cu") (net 4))
 (segment (start 160.0984 98.4786) (end 160.0984 93.8748) (width 0.4064) (layer "B.Cu") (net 4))
 (segment (start 137.6353 110.464225) (end 139.2229 110.464225) (width 0.4064) (layer "B.Cu") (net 14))
 (segment (start 140.4928 109.1942) (end 142.1026 109.1942) (width 0.4064) (layer "B.Cu") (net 14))
 (segment (start 139.2229 110.4641) (end 140.4928 109.1942) (width 0.4064) (layer "B.Cu") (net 14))
 (segment (start 139.2229 110.464225) (end 139.2229 110.4641) (width 0.4064) (layer "B.Cu") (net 14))
 (segment (start 142.1026 109.1942) (end 142.182 109.1148) (width 0.4064) (layer "B.Cu") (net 14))
 (segment (start 157.3278 112.2179) (end 157.3278 98.1136) (width 0.4064) (layer "F.Cu") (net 11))
 (segment (start 152.7078 95.2236) (end 150.7378 95.2236) (width 0.4064) (layer "F.Cu") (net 11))
 (segment (start 144.1678 117.8536) (end 160.2497 117.8536) (width 0.4064) (layer "F.Cu") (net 11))
 (segment (start 150.7378 95.2236) (end 148.9128 93.3986) (width 0.4064) (layer "F.Cu") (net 11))
 (segment (start 161.6066 116.4967) (end 157.3278 112.2179) (width 0.4064) (layer "F.Cu") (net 11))
 (segment (start 143.3507 93.3986) (end 143.3505 93.3988) (width 0.4064) (layer "F.Cu") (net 11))
 (segment (start 157.3278 98.1136) (end 158.1534 97.288) (width 0.4064) (layer "F.Cu") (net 11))
 (segment (start 157.3278 98.1136) (end 157.2678 98.0536) (width 0.4064) (layer "F.Cu") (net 11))
 (segment (start 155.5378 98.0536) (end 152.7078 95.2236) (width 0.4064) (layer "F.Cu") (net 11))
 (segment (start 157.2678 98.0536) (end 155.5378 98.0536) (width 0.4064) (layer "F.Cu") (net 11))
 (segment (start 158.1534 97.288) (end 161.9241 97.288) (width 0.4064) (layer "F.Cu") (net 11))
 (segment (start 160.2497 117.8536) (end 161.6066 116.4967) (width 0.4064) (layer "F.Cu") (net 11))
 (segment (start 148.9128 93.3986) (end 143.3507 93.3986) (width 0.4064) (layer "F.Cu") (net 11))
 (via (at 161.6066 116.4967) (size 1.4224) (drill 1) (layers "F.Cu" "B.Cu") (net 11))
 (via (at 144.1678 117.8536) (size 1.0064) (drill 0.6) (layers "F.Cu" "B.Cu") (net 11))
 (via (at 161.9241 97.288) (size 1.4224) (drill 1) (layers "F.Cu" "B.Cu") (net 11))
 (segment (start 142.635925 92.684225) (end 143.3505 93.3988) (width 0.4064) (layer "B.Cu") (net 11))
 (segment (start 144.1441 117.8299) (end 144.1441 111.0992) (width 0.4064) (layer "B.Cu") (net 11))
 (segment (start 144.1441 111.0992) (end 143.4297 110.3848) (width 0.4064) (layer "B.Cu") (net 11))
 (segment (start 143.4297 110.3848) (end 142.182 110.3848) (width 0.4064) (layer "B.Cu") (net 11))
 (segment (start 144.1678 117.8536) (end 144.1441 117.8299) (width 0.4064) (layer "B.Cu") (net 11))
 (segment (start 137.6353 93.23985) (end 138.190925 92.684225) (width 0.4064) (layer "B.Cu") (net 11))
 (segment (start 141.7628 94.9865) (end 143.3505 93.3988) (width 0.4064) (layer "B.Cu") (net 11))
 (segment (start 143.3505 93.3988) (end 143.3503 93.3986) (width 0.4064) (layer "B.Cu") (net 11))
 (segment (start 138.190925 92.684225) (end 142.635925 92.684225) (width 0.4064) (layer "B.Cu") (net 11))
 (segment (start 141.7628 102.7648) (end 141.7628 94.9865) (width 0.4064) (layer "B.Cu") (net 11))
 (segment (start 142.182 102.7648) (end 141.7628 102.7648) (width 0.4064) (layer "B.Cu") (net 11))
 (segment (start 137.6353 95.224225) (end 137.6353 93.23985) (width 0.4064) (layer "B.Cu") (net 11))
 (segment (start 146.6841 106.5748) (end 146.2873 106.1779) (width 0.4064) (layer "B.Cu") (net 20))
 (segment (start 146.2873 106.1779) (end 146.2873 101.6535) (width 0.4064) (layer "B.Cu") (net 20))
 (segment (start 149.3033 89.2712) (end 151.6848 89.2712) (width 0.4064) (layer "B.Cu") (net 20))
 (segment (start 147.0809 91.4936) (end 149.3033 89.2712) (width 0.4064) (layer "B.Cu") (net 20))
 (segment (start 147.0809 100.8599) (end 147.0809 91.4936) (width 0.4064) (layer "B.Cu") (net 20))
 (segment (start 146.2873 101.6535) (end 147.0809 100.8599) (width 0.4064) (layer "B.Cu") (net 20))
 (segment (start 146.6841 106.5748) (end 148.3288 106.5748) (width 0.4064) (layer "B.Cu") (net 20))
 (segment (start 145.2553 107.2098) (end 145.2553 101.1772) (width 0.4064) (layer "B.Cu") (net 19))
 (segment (start 151.7641 98.7167) (end 151.7641 99.5011) (width 0.4064) (layer "B.Cu") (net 19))
 (segment (start 150.0178 91.9698) (end 150.0178 96.9704) (width 0.4064) (layer "B.Cu") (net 19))
 (segment (start 146.2872 100.1454) (end 146.2872 89.3505) (width 0.4064) (layer "B.Cu") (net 19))
 (segment (start 150.0178 96.9704) (end 151.7641 98.7167) (width 0.4064) (layer "B.Cu") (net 19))
 (segment (start 145.8903 107.8448) (end 145.2553 107.2098) (width 0.4064) (layer "B.Cu") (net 19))
 (segment (start 150.8909 91.0967) (end 150.0178 91.9698) (width 0.4064) (layer "B.Cu") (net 19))
 (segment (start 146.2872 89.3505) (end 147.716 87.9217) (width 0.4064) (layer "B.Cu") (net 19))
 (segment (start 152.9547 90.6205) (end 152.4785 91.0967) (width 0.4064) (layer "B.Cu") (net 19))
 (segment (start 145.2553 101.1772) (end 146.2872 100.1454) (width 0.4064) (layer "B.Cu") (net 19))
 (segment (start 152.4784 87.9217) (end 152.9547 88.398) (width 0.4064) (layer "B.Cu") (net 19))
 (segment (start 152.9547 88.398) (end 152.9547 90.6205) (width 0.4064) (layer "B.Cu") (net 19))
 (segment (start 145.8903 107.8448) (end 148.3288 107.8448) (width 0.4064) (layer "B.Cu") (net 19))
 (segment (start 152.4785 91.0967) (end 150.8909 91.0967) (width 0.4064) (layer "B.Cu") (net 19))
 (segment (start 151.7641 99.5011) (end 151.7455 99.5197) (width 0.4064) (layer "B.Cu") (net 19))
 (segment (start 147.716 87.9217) (end 152.4784 87.9217) (width 0.4064) (layer "B.Cu") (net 19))
 (segment (start 151.2082 109.1235) (end 151.2082 109.1148) (width 0.4064) (layer "B.Cu") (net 21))
 (segment (start 151.7539 109.6692) (end 151.2082 109.1235) (width 0.4064) (layer "B.Cu") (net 21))
 (segment (start 151.2082 109.1148) (end 148.3288 109.1148) (width 0.4064) (layer "B.Cu") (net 21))
 (segment (start 151.9228 93.1605) (end 153.0341 93.1605) (width 0.4064) (layer "B.Cu") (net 7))
 (segment (start 154.2248 91.9698) (end 154.2248 89.2712) (width 0.4064) (layer "B.Cu") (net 7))
 (segment (start 151.764 93.1604) (end 151.9228 93.1605) (width 0.4064) (layer "B.Cu") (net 7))
 (segment (start 153.0341 93.1605) (end 154.2248 91.9698) (width 0.4064) (layer "B.Cu") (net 7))
 (segment (start 154.3041 101.9711) (end 154.3041 99.5383) (width 0.4064) (layer "B.Cu") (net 3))
 (segment (start 154.2247 102.0505) (end 154.2247 102.0504) (width 0.4064) (layer "B.Cu") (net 3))
 (segment (start 154.3041 99.5383) (end 154.2855 99.5197) (width 0.4064) (layer "B.Cu") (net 3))
 (segment (start 153.5104 102.6854) (end 154.2247 102.0505) (width 0.4064) (layer "B.Cu") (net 3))
 (segment (start 154.2247 102.0504) (end 154.3041 101.9711) (width 0.4064) (layer "B.Cu") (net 3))
 (segment (start 152.8752 113.3216) (end 154.304 112.0516) (width 0.4064) (layer "B.Cu") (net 10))
 (segment (start 154.304 109.6793) (end 154.2939 109.6692) (width 0.4064) (layer "B.Cu") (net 10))
 (segment (start 154.304 112.0516) (end 154.304 109.6793) (width 0.4064) (layer "B.Cu") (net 10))
 (segment (start 140.41345 103.5586) (end 140.41345 94.2717) (width 0.4064) (layer "B.Cu") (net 5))
 (segment (start 142.182 104.0348) (end 140.88965 104.0348) (width 0.4064) (layer "B.Cu") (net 5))
 (segment (start 140.88965 104.0348) (end 140.41345 103.5586) (width 0.4064) (layer "B.Cu") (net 5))
 (segment (start 148.5096 102.584) (end 148.5096 95.9386) (width 0.4064) (layer "B.Cu") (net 1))
 (segment (start 148.3288 102.7648) (end 148.5096 102.584) (width 0.4064) (layer "B.Cu") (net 1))
 (segment (start 151.129 104.0348) (end 148.3288 104.0348) (width 0.4064) (layer "B.Cu") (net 15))
 (segment (start 152.2402 105.1461) (end 151.8433 104.7491) (width 0.4064) (layer "B.Cu") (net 15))
 (segment (start 151.8433 104.7491) (end 151.129 104.0348) (width 0.4064) (layer "B.Cu") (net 15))
 (segment (start 153.1134 107.2098) (end 152.5578 106.6542) (width 0.4064) (layer "B.Cu") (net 8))
 (segment (start 151.5259 106.6542) (end 150.1765 105.3048) (width 0.4064) (layer "B.Cu") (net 8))
 (segment (start 150.9702 116.0998) (end 150.9702 112.7661) (width 0.4064) (layer "B.Cu") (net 8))
 (segment (start 150.1765 105.3048) (end 148.3288 105.3048) (width 0.4064) (layer "B.Cu") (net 8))
 (segment (start 152.5578 106.6542) (end 151.5259 106.6542) (width 0.4064) (layer "B.Cu") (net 8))
 (segment (start 153.1134 110.6229) (end 153.1134 107.2098) (width 0.4064) (layer "B.Cu") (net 8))
 (segment (start 150.9702 112.7661) (end 153.1134 110.6229) (width 0.4064) (layer "B.Cu") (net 8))
 (segment (start 156.9774 86.8898) (end 158.5971 88.5095) (width 0.4064) (layer "B.Cu") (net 6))
 (segment (start 140.41345 86.6517) (end 140.2547 86.8898) (width 0.4064) (layer "B.Cu") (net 6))
 (segment (start 140.2547 86.8898) (end 156.9774 86.8898) (width 0.4064) (layer "B.Cu") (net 6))
 (segment (start 158.5971 88.5095) (end 158.5971 89.3425) (width 0.4064) (layer "B.Cu") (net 6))
 (segment (start 158.5971 89.3425) (end 158.588 89.3516) (width 0.4064) (layer "B.Cu") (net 6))
 (segment (start 158.5904 99.5107) (end 158.5904 98.3993) (width 0.4064) (layer "B.Cu") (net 2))
 (segment (start 158.5904 98.3993) (end 156.1296 95.9386) (width 0.4064) (layer "B.Cu") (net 2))
 (segment (start 158.7491 109.5119) (end 158.7491 106.2573) (width 0.4064) (layer "B.Cu") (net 16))
 (segment (start 159.2254 105.7811) (end 159.8602 105.1461) (width 0.4064) (layer "B.Cu") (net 16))
 (segment (start 158.7491 106.2573) (end 159.2254 105.7811) (width 0.4064) (layer "B.Cu") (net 16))
 (segment (start 158.5904 109.6706) (end 158.7491 109.5119) (width 0.4064) (layer "B.Cu") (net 16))
 (segment (start 158.5902 119.8304) (end 158.5902 116.0998) (width 0.4064) (layer "B.Cu") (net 9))
 (segment (start 158.5904 119.8306) (end 158.5902 119.8304) (width 0.4064) (layer "B.Cu") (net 9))
 (segment (start 149.7797 110.3848) (end 148.3288 110.3848) (width 0.4064) (layer "B.Cu") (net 17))
 (segment (start 147.9541 114.0361) (end 148.5097 114.0361) (width 0.4064) (layer "B.Cu") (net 17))
 (segment (start 148.5097 114.0361) (end 150.1766 112.3692) (width 0.4064) (layer "B.Cu") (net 17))
 (segment (start 150.1766 112.3692) (end 150.1766 110.7817) (width 0.4064) (layer "B.Cu") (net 17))
 (segment (start 150.1766 110.7817) (end 149.7797 110.3848) (width 0.4064) (layer "B.Cu") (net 17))
 (segment (start 147.9541 121.6561) (end 147.9541 120.5448) (width 0.4064) (layer "B.Cu") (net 18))
 (segment (start 151.7709 119.9098) (end 151.7793 119.9182) (width 0.4064) (layer "B.Cu") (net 18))
 (segment (start 148.5891 119.9098) (end 151.7709 119.9098) (width 0.4064) (layer "B.Cu") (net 18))
 (segment (start 147.9541 120.5448) (end 148.5891 119.9098) (width 0.4064) (layer "B.Cu") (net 18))
 (segment (start 140.7309 105.3048) (end 142.182 105.3048) (width 0.4064) (layer "B.Cu") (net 13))
 (segment (start 138.2702 102.844225) (end 138.2702 102.8441) (width 0.4064) (layer "B.Cu") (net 13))
 (segment (start 138.2702 102.8441) (end 140.7309 105.3048) (width 0.4064) (layer "B.Cu") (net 13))
 (segment (start 137.6353 102.844225) (end 138.2702 102.844225) (width 0.4064) (layer "B.Cu") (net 13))
 (segment (start 137.6353 97.764225) (end 141.1673 97.764225) (width 0.4064) (layer "F.Cu") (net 12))
 (segment (start 141.0478 101.6436) (end 144.0878 101.6436) (width 0.4064) (layer "F.Cu") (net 12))
 (segment (start 144.0878 101.6436) (end 145.2478 100.4836) (width 0.4064) (layer "F.Cu") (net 12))
 (segment (start 141.1673 97.764225) (end 141.1673 97.7641) (width 0.4064) (layer "F.Cu") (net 12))
 (segment (start 144.1878 96.9636) (end 141.9678 96.9636) (width 0.4064) (layer "F.Cu") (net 12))
 (segment (start 140.2378 107.8636) (end 140.3778 107.7236) (width 0.4064) (layer "F.Cu") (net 12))
 (segment (start 140.3778 102.3136) (end 141.0478 101.6436) (width 0.4064) (layer "F.Cu") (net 12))
 (segment (start 141.9678 96.9636) (end 141.1673 97.7641) (width 0.4064) (layer "F.Cu") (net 12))
 (segment (start 145.2478 98.0236) (end 144.1878 96.9636) (width 0.4064) (layer "F.Cu") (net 12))
 (segment (start 140.3778 107.7236) (end 140.3778 102.3136) (width 0.4064) (layer "F.Cu") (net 12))
 (segment (start 145.2478 100.4836) (end 145.2478 98.0236) (width 0.4064) (layer "F.Cu") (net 12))
 (via (at 140.2378 107.8636) (size 1.0064) (drill 0.6) (layers "F.Cu" "B.Cu") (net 12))
 (segment (start 142.1632 107.8636) (end 140.2378 107.8636) (width 0.4064) (layer "B.Cu") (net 12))
 (segment (start 142.182 107.8448) (end 142.1632 107.8636) (width 0.4064) (layer "B.Cu") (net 12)))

